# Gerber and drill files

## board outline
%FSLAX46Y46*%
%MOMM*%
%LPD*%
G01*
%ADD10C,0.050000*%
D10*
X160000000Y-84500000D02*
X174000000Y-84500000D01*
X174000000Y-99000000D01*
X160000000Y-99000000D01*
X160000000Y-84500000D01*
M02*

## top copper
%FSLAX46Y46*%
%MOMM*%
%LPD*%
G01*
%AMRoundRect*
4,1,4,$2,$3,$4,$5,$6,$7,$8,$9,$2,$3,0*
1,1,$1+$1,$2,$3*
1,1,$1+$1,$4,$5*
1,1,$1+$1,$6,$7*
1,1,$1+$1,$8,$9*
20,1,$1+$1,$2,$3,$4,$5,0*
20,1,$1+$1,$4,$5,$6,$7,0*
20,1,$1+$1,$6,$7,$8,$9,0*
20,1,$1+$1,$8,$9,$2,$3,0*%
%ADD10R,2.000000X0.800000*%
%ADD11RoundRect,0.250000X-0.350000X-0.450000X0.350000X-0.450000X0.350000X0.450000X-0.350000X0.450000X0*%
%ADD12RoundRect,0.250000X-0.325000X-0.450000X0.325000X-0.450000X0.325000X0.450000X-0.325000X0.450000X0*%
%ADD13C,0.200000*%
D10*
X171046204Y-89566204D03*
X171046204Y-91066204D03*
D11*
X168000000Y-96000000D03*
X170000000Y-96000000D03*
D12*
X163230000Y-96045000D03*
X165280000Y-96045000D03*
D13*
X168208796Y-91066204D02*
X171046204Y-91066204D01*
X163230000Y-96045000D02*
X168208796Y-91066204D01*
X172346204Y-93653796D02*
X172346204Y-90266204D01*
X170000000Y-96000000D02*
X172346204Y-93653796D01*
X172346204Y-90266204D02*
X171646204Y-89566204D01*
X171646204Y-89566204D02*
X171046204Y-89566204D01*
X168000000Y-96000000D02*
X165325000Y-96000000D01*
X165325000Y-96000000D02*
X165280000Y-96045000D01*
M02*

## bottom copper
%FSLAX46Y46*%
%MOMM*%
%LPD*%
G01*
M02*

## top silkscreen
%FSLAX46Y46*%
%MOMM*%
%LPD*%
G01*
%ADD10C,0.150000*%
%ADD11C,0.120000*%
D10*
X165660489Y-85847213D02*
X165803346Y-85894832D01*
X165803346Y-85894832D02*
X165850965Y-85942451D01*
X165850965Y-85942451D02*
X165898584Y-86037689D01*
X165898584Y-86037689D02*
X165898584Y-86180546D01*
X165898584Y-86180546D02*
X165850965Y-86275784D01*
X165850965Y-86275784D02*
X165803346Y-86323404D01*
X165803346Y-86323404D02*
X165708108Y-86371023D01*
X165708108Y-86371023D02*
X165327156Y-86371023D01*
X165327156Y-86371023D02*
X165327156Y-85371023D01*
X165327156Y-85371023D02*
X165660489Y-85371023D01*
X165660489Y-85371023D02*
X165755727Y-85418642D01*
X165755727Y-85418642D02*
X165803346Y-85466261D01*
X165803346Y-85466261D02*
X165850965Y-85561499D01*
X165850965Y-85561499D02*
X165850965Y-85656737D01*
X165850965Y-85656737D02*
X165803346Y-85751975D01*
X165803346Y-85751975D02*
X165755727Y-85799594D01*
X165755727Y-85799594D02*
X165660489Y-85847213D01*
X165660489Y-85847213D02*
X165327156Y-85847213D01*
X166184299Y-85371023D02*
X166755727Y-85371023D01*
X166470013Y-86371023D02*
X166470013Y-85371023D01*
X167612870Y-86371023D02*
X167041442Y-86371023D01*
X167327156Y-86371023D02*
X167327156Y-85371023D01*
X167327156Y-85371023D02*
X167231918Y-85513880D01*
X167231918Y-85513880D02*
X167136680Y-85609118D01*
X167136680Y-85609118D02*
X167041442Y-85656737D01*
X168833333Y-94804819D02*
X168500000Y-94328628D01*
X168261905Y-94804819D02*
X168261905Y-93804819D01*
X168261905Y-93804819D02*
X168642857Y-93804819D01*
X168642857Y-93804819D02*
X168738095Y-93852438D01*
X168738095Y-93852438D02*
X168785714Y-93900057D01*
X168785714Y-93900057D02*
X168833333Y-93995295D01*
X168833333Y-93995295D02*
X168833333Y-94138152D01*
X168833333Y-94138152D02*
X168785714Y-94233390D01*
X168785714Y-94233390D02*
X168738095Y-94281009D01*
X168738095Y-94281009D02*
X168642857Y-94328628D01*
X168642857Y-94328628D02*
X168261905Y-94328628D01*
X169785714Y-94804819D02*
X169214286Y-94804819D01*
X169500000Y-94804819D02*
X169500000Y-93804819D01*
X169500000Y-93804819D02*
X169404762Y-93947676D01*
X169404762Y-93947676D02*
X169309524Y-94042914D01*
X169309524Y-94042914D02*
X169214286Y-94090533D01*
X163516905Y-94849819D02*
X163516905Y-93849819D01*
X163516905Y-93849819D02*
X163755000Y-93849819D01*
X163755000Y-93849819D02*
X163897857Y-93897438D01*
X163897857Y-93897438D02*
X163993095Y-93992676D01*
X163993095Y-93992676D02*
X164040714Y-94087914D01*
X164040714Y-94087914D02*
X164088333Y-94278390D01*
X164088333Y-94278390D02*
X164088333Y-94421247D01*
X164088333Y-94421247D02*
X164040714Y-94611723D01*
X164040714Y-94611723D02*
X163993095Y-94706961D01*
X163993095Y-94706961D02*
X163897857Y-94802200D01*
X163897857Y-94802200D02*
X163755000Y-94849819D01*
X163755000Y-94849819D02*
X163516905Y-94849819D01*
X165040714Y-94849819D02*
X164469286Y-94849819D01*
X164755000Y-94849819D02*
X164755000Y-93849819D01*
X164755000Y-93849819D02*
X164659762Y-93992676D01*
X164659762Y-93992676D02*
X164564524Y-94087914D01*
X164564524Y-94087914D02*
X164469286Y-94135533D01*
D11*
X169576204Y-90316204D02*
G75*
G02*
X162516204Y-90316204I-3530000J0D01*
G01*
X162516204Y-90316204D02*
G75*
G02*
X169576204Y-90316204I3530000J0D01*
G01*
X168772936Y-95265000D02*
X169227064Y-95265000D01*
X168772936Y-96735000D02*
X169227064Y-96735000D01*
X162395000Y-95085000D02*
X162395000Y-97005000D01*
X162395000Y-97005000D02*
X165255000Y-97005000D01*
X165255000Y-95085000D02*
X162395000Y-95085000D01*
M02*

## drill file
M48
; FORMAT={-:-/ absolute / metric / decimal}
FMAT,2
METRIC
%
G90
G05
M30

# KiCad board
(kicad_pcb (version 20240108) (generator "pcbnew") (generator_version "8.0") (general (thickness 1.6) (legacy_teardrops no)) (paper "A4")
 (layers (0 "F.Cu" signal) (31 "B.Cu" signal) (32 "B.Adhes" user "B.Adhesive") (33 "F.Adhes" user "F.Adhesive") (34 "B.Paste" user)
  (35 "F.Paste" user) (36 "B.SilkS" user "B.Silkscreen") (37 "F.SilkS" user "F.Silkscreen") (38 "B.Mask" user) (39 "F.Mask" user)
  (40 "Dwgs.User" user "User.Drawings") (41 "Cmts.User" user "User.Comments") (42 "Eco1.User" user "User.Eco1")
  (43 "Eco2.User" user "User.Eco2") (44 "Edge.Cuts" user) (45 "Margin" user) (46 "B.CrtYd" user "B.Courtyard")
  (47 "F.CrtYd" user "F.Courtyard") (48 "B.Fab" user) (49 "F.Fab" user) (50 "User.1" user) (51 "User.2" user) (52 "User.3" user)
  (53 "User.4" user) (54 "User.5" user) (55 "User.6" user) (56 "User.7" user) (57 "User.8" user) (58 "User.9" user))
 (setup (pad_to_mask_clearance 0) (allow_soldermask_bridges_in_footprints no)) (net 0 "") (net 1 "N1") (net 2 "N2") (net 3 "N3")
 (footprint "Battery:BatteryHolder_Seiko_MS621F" (layer "F.Cu") (at 171.046204 90.316204)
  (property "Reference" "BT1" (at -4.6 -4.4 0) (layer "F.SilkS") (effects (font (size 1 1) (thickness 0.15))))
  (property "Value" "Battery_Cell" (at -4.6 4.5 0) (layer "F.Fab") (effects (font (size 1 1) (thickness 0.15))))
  (fp_circle (center -5 0) (end -1.47 0) (stroke (width 0.12) (type solid)) (fill none) (layer "F.SilkS"))
  (pad "1" smd rect (at 0 -0.75) (size 2 0.8) (layers "F.Cu" "F.Paste" "F.Mask") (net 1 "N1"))
  (pad "2" smd rect (at 0 0.75) (size 2 0.8) (layers "F.Cu" "F.Paste" "F.Mask") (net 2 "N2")))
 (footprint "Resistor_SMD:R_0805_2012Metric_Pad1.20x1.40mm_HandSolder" (layer "F.Cu") (at 169 96)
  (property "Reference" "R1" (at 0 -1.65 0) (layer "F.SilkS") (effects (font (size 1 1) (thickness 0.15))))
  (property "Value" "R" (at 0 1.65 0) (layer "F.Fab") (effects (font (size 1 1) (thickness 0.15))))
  (fp_line (start -0.227064 -0.735) (end 0.227064 -0.735) (stroke (width 0.12) (type solid)) (layer "F.SilkS"))
  (fp_line (start -0.227064 0.735) (end 0.227064 0.735) (stroke (width 0.12) (type solid)) (layer "F.SilkS"))
  (pad "1" smd roundrect (at -1 0) (size 1.2 1.4) (layers "F.Cu" "F.Paste" "F.Mask") (roundrect_rratio 0.208333) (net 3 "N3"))
  (pad "2" smd roundrect (at 1 0) (size 1.2 1.4) (layers "F.Cu" "F.Paste" "F.Mask") (roundrect_rratio 0.208333) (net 1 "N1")))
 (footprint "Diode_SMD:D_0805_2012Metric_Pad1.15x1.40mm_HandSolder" (layer "F.Cu") (at 164.255 96.045)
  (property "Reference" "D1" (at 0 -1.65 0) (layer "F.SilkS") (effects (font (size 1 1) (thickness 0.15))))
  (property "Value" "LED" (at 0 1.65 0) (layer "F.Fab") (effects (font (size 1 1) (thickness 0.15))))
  (fp_line (start -1.86 -0.96) (end -1.86 0.96) (stroke (width 0.12) (type solid)) (layer "F.SilkS"))
  (fp_line (start -1.86 0.96) (end 1 0.96) (stroke (width 0.12) (type solid)) (layer "F.SilkS"))
  (fp_line (start 1 -0.96) (end -1.86 -0.96) (stroke (width 0.12) (type solid)) (layer "F.SilkS"))
  (pad "1" smd roundrect (at -1.025 0) (size 1.15 1.4) (layers "F.Cu" "F.Paste" "F.Mask") (roundrect_rratio 0.217391) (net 2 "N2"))
  (pad "2" smd roundrect (at 1.025 0) (size 1.15 1.4) (layers "F.Cu" "F.Paste" "F.Mask") (roundrect_rratio 0.217391) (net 3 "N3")))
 (gr_rect (start 160 84.5) (end 174 99) (stroke (width 0.05) (type default)) (fill none) (layer "Edge.Cuts"))
 (segment (start 168.208796 91.066204) (end 171.046204 91.066204) (width 0.2) (layer "F.Cu") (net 2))
 (segment (start 163.23 96.045) (end 168.208796 91.066204) (width 0.2) (layer "F.Cu") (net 2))
 (segment (start 172.346204 93.653796) (end 172.346204 90.266204) (width 0.2) (layer "F.Cu") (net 1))
 (segment (start 170 96) (end 172.346204 93.653796) (width 0.2) (layer "F.Cu") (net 1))
 (segment (start 172.346204 90.266204) (end 171.646204 89.566204) (width 0.2) (layer "F.Cu") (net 1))
 (segment (start 171.646204 89.566204) (end 171.046204 89.566204) (width 0.2) (layer "F.Cu") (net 1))
 (segment (start 168 96) (end 165.325 96) (width 0.2) (layer "F.Cu") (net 3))
 (segment (start 165.325 96) (end 165.28 96.045) (width 0.2) (layer "F.Cu") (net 3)))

